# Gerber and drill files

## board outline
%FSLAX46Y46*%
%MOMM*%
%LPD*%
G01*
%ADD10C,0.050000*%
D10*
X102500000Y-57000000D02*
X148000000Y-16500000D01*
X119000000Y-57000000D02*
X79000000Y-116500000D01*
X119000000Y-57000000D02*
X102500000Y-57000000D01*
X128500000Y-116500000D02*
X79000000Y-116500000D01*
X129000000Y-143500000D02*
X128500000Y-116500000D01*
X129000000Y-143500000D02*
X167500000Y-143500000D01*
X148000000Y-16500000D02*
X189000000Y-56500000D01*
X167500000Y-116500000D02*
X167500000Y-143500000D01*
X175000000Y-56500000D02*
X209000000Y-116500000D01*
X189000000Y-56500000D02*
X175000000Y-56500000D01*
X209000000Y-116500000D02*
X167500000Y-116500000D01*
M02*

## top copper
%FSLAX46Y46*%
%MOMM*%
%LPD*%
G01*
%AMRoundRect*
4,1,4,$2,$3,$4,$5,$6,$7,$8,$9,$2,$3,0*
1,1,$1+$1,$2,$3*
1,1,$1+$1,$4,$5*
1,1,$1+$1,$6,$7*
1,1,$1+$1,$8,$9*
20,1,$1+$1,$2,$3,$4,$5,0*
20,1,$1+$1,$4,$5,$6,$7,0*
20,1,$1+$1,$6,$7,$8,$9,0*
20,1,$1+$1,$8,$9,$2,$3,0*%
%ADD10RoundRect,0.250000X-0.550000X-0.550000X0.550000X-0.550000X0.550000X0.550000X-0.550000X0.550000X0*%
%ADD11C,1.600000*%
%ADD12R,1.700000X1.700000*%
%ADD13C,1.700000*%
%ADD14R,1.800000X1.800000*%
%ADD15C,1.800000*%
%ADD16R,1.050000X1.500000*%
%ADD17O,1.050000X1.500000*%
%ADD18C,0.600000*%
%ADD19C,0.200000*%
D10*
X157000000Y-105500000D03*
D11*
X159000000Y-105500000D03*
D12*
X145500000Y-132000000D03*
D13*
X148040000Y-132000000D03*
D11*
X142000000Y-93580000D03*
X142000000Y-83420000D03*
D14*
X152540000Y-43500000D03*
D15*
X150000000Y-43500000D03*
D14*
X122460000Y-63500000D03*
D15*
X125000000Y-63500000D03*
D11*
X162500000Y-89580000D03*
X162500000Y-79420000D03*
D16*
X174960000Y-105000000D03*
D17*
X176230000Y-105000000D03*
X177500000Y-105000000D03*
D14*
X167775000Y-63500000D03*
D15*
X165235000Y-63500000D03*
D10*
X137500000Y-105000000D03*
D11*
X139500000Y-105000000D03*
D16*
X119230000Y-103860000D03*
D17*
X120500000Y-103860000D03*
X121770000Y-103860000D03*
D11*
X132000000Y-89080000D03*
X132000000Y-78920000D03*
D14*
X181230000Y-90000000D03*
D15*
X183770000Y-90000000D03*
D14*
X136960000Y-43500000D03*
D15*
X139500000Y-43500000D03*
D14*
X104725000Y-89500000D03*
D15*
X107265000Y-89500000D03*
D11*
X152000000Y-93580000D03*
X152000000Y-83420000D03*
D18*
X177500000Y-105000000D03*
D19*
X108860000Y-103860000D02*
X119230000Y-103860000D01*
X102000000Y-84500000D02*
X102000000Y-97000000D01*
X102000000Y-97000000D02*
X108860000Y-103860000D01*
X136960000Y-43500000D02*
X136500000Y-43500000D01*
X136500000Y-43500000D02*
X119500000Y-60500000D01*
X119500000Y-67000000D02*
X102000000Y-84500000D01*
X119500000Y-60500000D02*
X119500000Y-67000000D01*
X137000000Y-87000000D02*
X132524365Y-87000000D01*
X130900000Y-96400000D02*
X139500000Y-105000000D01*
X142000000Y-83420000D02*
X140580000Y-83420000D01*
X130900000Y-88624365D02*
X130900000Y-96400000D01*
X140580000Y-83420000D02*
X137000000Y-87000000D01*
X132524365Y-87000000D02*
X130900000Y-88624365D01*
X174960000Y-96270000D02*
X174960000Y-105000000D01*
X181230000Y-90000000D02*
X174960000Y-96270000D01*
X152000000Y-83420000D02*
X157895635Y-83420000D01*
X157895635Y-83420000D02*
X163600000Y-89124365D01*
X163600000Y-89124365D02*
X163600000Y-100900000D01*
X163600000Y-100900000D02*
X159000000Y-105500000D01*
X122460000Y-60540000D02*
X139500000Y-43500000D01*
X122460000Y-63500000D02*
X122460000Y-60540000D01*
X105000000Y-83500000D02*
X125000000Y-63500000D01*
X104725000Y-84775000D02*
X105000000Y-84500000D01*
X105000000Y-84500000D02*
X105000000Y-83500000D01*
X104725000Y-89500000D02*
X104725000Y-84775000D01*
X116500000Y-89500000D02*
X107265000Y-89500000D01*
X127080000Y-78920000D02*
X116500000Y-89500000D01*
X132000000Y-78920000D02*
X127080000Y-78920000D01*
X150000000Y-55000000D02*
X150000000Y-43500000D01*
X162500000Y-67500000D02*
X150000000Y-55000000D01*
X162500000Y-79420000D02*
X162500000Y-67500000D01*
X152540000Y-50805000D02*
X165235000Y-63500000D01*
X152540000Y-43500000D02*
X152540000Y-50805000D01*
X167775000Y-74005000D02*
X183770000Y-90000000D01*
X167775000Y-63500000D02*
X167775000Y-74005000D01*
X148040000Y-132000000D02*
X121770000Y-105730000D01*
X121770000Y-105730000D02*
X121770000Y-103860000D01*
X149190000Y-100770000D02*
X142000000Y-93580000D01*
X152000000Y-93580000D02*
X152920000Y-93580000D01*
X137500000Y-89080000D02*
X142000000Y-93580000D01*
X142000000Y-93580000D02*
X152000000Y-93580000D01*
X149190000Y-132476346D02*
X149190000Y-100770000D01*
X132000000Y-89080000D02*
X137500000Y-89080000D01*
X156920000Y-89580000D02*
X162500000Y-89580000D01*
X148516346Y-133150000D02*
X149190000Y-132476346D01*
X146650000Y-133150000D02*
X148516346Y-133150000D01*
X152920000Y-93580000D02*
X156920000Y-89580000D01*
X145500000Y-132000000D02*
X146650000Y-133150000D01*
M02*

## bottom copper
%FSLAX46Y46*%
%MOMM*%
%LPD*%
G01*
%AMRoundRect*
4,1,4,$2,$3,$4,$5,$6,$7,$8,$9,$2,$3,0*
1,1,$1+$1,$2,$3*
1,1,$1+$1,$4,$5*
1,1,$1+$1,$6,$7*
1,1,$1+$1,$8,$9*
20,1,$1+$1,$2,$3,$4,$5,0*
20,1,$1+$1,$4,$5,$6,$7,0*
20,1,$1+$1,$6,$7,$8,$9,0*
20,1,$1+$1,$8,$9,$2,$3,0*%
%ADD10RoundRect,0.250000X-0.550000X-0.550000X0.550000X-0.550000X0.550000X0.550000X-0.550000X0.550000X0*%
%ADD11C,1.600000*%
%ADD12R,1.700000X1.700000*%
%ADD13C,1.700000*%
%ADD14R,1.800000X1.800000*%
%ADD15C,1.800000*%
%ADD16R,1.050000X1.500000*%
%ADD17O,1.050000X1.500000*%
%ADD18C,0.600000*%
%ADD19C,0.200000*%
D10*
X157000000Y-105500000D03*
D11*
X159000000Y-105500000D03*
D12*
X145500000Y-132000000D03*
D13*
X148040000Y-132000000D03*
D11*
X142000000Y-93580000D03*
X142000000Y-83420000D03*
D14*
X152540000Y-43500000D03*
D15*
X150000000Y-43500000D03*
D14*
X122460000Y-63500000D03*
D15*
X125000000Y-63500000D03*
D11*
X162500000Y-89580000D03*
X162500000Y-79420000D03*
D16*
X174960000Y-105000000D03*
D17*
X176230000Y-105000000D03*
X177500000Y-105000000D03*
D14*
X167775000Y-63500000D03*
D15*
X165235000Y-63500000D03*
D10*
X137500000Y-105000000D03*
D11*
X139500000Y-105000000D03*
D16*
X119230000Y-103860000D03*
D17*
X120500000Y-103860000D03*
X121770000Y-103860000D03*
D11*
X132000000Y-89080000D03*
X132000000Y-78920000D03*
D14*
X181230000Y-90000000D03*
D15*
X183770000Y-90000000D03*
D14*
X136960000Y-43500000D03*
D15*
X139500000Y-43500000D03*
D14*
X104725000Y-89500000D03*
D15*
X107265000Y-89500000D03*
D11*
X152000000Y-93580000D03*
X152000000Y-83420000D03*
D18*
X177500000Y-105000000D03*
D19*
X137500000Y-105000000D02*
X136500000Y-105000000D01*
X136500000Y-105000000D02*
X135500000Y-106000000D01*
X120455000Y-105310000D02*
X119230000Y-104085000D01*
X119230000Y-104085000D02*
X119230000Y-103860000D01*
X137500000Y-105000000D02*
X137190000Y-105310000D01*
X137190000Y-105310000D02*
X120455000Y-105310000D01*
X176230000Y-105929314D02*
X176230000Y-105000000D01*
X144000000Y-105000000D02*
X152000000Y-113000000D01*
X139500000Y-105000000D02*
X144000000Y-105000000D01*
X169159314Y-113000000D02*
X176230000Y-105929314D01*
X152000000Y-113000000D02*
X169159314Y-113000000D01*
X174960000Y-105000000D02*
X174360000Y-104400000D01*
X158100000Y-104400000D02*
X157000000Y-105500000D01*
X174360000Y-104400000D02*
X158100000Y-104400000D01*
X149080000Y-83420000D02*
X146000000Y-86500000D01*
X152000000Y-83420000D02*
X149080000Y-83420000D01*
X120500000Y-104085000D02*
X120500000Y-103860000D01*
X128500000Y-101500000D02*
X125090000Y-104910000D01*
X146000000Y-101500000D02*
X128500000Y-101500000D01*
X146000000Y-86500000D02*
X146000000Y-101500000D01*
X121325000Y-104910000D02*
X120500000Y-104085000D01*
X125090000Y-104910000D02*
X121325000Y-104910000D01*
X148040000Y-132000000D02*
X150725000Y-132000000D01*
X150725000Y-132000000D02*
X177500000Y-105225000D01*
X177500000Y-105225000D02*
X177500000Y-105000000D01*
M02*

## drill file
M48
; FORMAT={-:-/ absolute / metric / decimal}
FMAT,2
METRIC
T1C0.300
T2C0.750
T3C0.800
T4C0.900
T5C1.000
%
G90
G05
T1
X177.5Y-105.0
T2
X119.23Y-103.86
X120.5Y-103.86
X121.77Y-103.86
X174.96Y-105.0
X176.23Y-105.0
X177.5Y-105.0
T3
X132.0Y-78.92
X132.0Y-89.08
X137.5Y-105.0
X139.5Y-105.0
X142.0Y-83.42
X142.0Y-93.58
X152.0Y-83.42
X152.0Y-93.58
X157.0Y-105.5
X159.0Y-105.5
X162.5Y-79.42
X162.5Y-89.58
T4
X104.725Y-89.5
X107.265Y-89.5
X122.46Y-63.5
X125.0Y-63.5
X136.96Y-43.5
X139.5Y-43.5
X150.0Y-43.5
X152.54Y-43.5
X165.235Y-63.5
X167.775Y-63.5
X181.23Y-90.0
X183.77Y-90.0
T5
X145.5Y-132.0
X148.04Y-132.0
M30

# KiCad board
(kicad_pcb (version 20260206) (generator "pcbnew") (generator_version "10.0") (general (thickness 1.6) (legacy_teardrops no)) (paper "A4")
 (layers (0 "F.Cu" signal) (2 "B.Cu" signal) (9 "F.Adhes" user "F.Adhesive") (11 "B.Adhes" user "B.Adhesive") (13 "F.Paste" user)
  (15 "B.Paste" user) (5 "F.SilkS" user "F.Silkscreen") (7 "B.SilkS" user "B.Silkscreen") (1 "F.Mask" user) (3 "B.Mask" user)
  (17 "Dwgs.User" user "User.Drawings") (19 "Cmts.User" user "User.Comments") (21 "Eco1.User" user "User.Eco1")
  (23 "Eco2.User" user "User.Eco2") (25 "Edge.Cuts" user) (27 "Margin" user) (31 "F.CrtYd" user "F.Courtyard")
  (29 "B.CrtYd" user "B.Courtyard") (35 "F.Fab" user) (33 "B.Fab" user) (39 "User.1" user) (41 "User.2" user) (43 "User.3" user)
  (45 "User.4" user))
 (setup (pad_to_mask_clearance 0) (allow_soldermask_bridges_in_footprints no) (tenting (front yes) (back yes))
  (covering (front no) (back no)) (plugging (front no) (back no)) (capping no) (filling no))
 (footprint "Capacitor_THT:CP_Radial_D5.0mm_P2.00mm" (layer "F.Cu") (at 157 105.5)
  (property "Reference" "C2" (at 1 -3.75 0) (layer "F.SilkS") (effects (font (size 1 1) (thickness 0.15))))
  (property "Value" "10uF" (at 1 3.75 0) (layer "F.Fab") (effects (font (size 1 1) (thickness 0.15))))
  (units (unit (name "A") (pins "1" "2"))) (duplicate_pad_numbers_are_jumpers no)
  (pad "1" thru_hole roundrect (at 0 0) (size 1.6 1.6) (drill 0.8) (layers "*.Cu" "*.Mask") (remove_unused_layers no)
   (roundrect_rratio 0.15625) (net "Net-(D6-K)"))
  (pad "2" thru_hole circle (at 2 0) (size 1.6 1.6) (drill 0.8) (layers "*.Cu" "*.Mask") (remove_unused_layers no) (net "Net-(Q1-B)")))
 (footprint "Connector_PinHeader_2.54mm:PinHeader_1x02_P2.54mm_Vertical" (layer "F.Cu") (at 145.5 132 90)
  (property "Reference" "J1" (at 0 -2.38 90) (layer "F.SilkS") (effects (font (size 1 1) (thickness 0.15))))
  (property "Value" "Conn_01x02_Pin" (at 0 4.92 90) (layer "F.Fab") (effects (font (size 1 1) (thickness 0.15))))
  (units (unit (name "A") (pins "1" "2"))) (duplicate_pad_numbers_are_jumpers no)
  (pad "1" thru_hole rect (at 0 0 90) (size 1.7 1.7) (drill 1) (layers "*.Cu" "*.Mask") (remove_unused_layers no) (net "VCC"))
  (pad "2" thru_hole circle (at 0 2.54 90) (size 1.7 1.7) (drill 1) (layers "*.Cu" "*.Mask") (remove_unused_layers no) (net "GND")))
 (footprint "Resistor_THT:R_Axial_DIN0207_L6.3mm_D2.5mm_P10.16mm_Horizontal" (layer "F.Cu") (at 142 93.58 90)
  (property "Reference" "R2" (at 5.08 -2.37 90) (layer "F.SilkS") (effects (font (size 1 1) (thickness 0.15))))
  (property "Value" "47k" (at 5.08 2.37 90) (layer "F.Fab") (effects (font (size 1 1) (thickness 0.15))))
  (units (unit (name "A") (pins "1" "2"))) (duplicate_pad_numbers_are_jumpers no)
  (pad "1" thru_hole circle (at 0 0 90) (size 1.6 1.6) (drill 0.8) (layers "*.Cu" "*.Mask") (remove_unused_layers no) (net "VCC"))
  (pad "2" thru_hole circle (at 10.16 0 90) (size 1.6 1.6) (drill 0.8) (layers "*.Cu" "*.Mask") (remove_unused_layers no) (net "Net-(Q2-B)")))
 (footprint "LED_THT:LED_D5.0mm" (layer "F.Cu") (at 152.54 43.5 180)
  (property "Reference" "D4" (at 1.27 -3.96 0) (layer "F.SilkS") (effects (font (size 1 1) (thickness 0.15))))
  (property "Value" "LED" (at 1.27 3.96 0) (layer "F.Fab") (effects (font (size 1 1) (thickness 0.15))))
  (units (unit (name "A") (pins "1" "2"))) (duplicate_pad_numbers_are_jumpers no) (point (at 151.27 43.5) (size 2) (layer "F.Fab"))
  (pad "1" thru_hole rect (at 0 0 180) (size 1.8 1.8) (drill 0.9) (layers "*.Cu" "*.Mask") (remove_unused_layers no) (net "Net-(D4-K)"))
  (pad "2" thru_hole circle (at 2.54 0 180) (size 1.8 1.8) (drill 0.9) (layers "*.Cu" "*.Mask") (remove_unused_layers no) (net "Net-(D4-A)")))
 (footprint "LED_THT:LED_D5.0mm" (layer "F.Cu") (at 122.46 63.5)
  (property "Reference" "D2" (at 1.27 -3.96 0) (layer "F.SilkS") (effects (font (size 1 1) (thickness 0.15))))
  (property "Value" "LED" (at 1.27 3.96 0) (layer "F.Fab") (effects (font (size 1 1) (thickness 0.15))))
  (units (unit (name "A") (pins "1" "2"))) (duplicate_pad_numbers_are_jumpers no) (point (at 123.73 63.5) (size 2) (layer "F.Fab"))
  (pad "1" thru_hole rect (at 0 0) (size 1.8 1.8) (drill 0.9) (layers "*.Cu" "*.Mask") (remove_unused_layers no) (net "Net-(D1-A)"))
  (pad "2" thru_hole circle (at 2.54 0) (size 1.8 1.8) (drill 0.9) (layers "*.Cu" "*.Mask") (remove_unused_layers no) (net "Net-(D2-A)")))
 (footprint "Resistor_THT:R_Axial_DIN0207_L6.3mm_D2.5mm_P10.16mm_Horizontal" (layer "F.Cu") (at 162.5 89.58 90)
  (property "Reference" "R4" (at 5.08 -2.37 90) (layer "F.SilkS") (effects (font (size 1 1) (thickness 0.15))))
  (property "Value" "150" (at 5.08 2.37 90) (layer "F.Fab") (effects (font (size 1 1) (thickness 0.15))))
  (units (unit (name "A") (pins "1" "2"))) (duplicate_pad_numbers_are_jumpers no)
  (pad "1" thru_hole circle (at 0 0 90) (size 1.6 1.6) (drill 0.8) (layers "*.Cu" "*.Mask") (remove_unused_layers no) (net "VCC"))
  (pad "2" thru_hole circle (at 10.16 0 90) (size 1.6 1.6) (drill 0.8) (layers "*.Cu" "*.Mask") (remove_unused_layers no) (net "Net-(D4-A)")))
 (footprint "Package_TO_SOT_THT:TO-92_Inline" (layer "F.Cu") (at 174.96 105)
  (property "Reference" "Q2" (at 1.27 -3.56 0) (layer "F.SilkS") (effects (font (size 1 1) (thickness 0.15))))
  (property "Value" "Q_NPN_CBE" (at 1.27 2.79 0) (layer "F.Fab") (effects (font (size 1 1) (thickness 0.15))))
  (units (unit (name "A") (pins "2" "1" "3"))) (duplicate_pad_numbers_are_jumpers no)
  (pad "1" thru_hole rect (at 0 0) (size 1.05 1.5) (drill 0.75) (layers "*.Cu" "*.Mask") (remove_unused_layers no) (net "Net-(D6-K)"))
  (pad "2" thru_hole oval (at 1.27 0) (size 1.05 1.5) (drill 0.75) (layers "*.Cu" "*.Mask") (remove_unused_layers no) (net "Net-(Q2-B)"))
  (pad "3" thru_hole oval (at 2.54 0) (size 1.05 1.5) (drill 0.75) (layers "*.Cu" "*.Mask") (remove_unused_layers no) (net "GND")))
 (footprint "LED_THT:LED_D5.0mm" (layer "F.Cu") (at 167.775 63.5 180)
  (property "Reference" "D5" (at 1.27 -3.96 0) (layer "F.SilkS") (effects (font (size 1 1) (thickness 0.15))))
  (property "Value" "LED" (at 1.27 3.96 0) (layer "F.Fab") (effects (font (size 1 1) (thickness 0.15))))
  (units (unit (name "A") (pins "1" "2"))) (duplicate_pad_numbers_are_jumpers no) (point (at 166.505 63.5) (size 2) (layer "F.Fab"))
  (pad "1" thru_hole rect (at 0 0 180) (size 1.8 1.8) (drill 0.9) (layers "*.Cu" "*.Mask") (remove_unused_layers no) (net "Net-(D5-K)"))
  (pad "2" thru_hole circle (at 2.54 0 180) (size 1.8 1.8) (drill 0.9) (layers "*.Cu" "*.Mask") (remove_unused_layers no) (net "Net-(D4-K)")))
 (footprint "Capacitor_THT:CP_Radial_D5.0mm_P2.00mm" (layer "F.Cu") (at 137.5 105)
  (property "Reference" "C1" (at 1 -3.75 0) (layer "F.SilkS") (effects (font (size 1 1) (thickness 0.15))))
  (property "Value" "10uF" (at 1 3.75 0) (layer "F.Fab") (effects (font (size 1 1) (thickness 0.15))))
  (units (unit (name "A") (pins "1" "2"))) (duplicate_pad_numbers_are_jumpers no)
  (pad "1" thru_hole roundrect (at 0 0) (size 1.6 1.6) (drill 0.8) (layers "*.Cu" "*.Mask") (remove_unused_layers no)
   (roundrect_rratio 0.15625) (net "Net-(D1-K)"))
  (pad "2" thru_hole circle (at 2 0) (size 1.6 1.6) (drill 0.8) (layers "*.Cu" "*.Mask") (remove_unused_layers no) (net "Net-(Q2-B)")))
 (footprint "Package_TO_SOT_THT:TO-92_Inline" (layer "F.Cu") (at 119.23 103.86)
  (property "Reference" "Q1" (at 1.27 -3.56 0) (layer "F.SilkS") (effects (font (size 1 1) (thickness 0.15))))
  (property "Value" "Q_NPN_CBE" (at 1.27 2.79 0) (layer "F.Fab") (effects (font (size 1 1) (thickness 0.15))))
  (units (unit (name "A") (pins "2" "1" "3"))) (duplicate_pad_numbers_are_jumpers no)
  (pad "1" thru_hole rect (at 0 0) (size 1.05 1.5) (drill 0.75) (layers "*.Cu" "*.Mask") (remove_unused_layers no) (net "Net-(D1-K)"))
  (pad "2" thru_hole oval (at 1.27 0) (size 1.05 1.5) (drill 0.75) (layers "*.Cu" "*.Mask") (remove_unused_layers no) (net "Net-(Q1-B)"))
  (pad "3" thru_hole oval (at 2.54 0) (size 1.05 1.5) (drill 0.75) (layers "*.Cu" "*.Mask") (remove_unused_layers no) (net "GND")))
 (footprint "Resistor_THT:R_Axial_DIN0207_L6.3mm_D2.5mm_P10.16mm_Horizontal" (layer "F.Cu") (at 132 89.08 90)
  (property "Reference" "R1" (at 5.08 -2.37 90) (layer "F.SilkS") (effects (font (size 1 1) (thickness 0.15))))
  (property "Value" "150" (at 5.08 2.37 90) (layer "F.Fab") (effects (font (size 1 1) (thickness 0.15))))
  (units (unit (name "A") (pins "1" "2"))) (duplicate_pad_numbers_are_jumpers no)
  (pad "1" thru_hole circle (at 0 0 90) (size 1.6 1.6) (drill 0.8) (layers "*.Cu" "*.Mask") (remove_unused_layers no) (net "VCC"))
  (pad "2" thru_hole circle (at 10.16 0 90) (size 1.6 1.6) (drill 0.8) (layers "*.Cu" "*.Mask") (remove_unused_layers no) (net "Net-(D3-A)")))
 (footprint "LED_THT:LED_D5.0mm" (layer "F.Cu") (at 181.23 90)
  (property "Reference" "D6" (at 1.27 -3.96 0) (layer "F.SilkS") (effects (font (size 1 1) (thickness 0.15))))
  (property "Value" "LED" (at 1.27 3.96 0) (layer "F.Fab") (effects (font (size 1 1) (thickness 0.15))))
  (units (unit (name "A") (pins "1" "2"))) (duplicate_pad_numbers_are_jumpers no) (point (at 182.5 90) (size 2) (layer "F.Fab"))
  (pad "1" thru_hole rect (at 0 0) (size 1.8 1.8) (drill 0.9) (layers "*.Cu" "*.Mask") (remove_unused_layers no) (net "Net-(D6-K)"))
  (pad "2" thru_hole circle (at 2.54 0) (size 1.8 1.8) (drill 0.9) (layers "*.Cu" "*.Mask") (remove_unused_layers no) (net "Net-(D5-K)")))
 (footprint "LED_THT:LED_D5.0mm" (layer "F.Cu") (at 136.96 43.5)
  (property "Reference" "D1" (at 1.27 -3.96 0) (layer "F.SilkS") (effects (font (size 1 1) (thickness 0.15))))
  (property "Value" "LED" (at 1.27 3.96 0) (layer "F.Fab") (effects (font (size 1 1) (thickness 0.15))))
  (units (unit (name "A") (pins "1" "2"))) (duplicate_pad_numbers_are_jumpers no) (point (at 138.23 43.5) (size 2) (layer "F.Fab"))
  (pad "1" thru_hole rect (at 0 0) (size 1.8 1.8) (drill 0.9) (layers "*.Cu" "*.Mask") (remove_unused_layers no) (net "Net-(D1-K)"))
  (pad "2" thru_hole circle (at 2.54 0) (size 1.8 1.8) (drill 0.9) (layers "*.Cu" "*.Mask") (remove_unused_layers no) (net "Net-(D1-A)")))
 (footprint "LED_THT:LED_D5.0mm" (layer "F.Cu") (at 104.725 89.5)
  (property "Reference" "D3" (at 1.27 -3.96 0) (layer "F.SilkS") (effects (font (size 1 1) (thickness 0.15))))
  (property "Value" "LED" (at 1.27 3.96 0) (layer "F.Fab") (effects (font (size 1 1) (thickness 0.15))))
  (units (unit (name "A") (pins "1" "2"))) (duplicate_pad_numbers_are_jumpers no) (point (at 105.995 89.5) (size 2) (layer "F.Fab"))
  (pad "1" thru_hole rect (at 0 0) (size 1.8 1.8) (drill 0.9) (layers "*.Cu" "*.Mask") (remove_unused_layers no) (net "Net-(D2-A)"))
  (pad "2" thru_hole circle (at 2.54 0) (size 1.8 1.8) (drill 0.9) (layers "*.Cu" "*.Mask") (remove_unused_layers no) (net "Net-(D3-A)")))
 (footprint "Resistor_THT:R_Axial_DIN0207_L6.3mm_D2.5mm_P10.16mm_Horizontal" (layer "F.Cu") (at 152 93.58 90)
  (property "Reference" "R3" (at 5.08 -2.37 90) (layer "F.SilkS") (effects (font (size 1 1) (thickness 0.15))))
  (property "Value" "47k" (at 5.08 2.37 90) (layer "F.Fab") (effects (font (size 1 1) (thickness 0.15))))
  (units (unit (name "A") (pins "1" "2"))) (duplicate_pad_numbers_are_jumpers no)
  (pad "1" thru_hole circle (at 0 0 90) (size 1.6 1.6) (drill 0.8) (layers "*.Cu" "*.Mask") (remove_unused_layers no) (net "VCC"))
  (pad "2" thru_hole circle (at 10.16 0 90) (size 1.6 1.6) (drill 0.8) (layers "*.Cu" "*.Mask") (remove_unused_layers no) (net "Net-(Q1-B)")))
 (gr_line (start 102.5 57) (end 148 16.5) (stroke (width 0.05) (type default)) (layer "Edge.Cuts"))
 (gr_line (start 119 57) (end 79 116.5) (stroke (width 0.05) (type default)) (layer "Edge.Cuts"))
 (gr_line (start 119 57) (end 102.5 57) (stroke (width 0.05) (type default)) (layer "Edge.Cuts"))
 (gr_line (start 128.5 116.5) (end 79 116.5) (stroke (width 0.05) (type default)) (layer "Edge.Cuts"))
 (gr_line (start 129 143.5) (end 128.5 116.5) (stroke (width 0.05) (type default)) (layer "Edge.Cuts"))
 (gr_line (start 129 143.5) (end 167.5 143.5) (stroke (width 0.05) (type default)) (layer "Edge.Cuts"))
 (gr_line (start 148 16.5) (end 189 56.5) (stroke (width 0.05) (type default)) (layer "Edge.Cuts"))
 (gr_line (start 167.5 116.5) (end 167.5 143.5) (stroke (width 0.05) (type default)) (layer "Edge.Cuts"))
 (gr_line (start 175 56.5) (end 209 116.5) (stroke (width 0.05) (type default)) (layer "Edge.Cuts"))
 (gr_line (start 189 56.5) (end 175 56.5) (stroke (width 0.05) (type default)) (layer "Edge.Cuts"))
 (gr_line (start 209 116.5) (end 167.5 116.5) (stroke (width 0.05) (type default)) (layer "Edge.Cuts"))
 (segment (start 108.86 103.86) (end 119.23 103.86) (width 0.2) (layer "F.Cu") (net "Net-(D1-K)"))
 (segment (start 102 84.5) (end 102 97) (width 0.2) (layer "F.Cu") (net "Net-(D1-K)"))
 (segment (start 102 97) (end 108.86 103.86) (width 0.2) (layer "F.Cu") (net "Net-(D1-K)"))
 (segment (start 136.96 43.5) (end 136.5 43.5) (width 0.2) (layer "F.Cu") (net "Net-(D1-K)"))
 (segment (start 136.5 43.5) (end 119.5 60.5) (width 0.2) (layer "F.Cu") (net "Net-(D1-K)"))
 (segment (start 119.5 67) (end 102 84.5) (width 0.2) (layer "F.Cu") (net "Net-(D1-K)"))
 (segment (start 119.5 60.5) (end 119.5 67) (width 0.2) (layer "F.Cu") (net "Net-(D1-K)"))
 (segment (start 137.5 105) (end 136.5 105) (width 0.2) (layer "B.Cu") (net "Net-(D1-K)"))
 (segment (start 136.5 105) (end 135.5 106) (width 0.2) (layer "B.Cu") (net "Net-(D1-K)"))
 (segment (start 120.455 105.31) (end 119.23 104.085) (width 0.2) (layer "B.Cu") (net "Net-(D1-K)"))
 (segment (start 119.23 104.085) (end 119.23 103.86) (width 0.2) (layer "B.Cu") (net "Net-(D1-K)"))
 (segment (start 137.5 105) (end 137.19 105.31) (width 0.2) (layer "B.Cu") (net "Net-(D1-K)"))
 (segment (start 137.19 105.31) (end 120.455 105.31) (width 0.2) (layer "B.Cu") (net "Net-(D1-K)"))
 (segment (start 137 87) (end 132.524365 87) (width 0.2) (layer "F.Cu") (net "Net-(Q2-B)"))
 (segment (start 130.9 96.4) (end 139.5 105) (width 0.2) (layer "F.Cu") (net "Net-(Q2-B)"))
 (segment (start 142 83.42) (end 140.58 83.42) (width 0.2) (layer "F.Cu") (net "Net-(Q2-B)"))
 (segment (start 130.9 88.624365) (end 130.9 96.4) (width 0.2) (layer "F.Cu") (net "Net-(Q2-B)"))
 (segment (start 140.58 83.42) (end 137 87) (width 0.2) (layer "F.Cu") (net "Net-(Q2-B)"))
 (segment (start 132.524365 87) (end 130.9 88.624365) (width 0.2) (layer "F.Cu") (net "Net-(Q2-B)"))
 (segment (start 176.23 105.929314) (end 176.23 105) (width 0.2) (layer "B.Cu") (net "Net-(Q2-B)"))
 (segment (start 144 105) (end 152 113) (width 0.2) (layer "B.Cu") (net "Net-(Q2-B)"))
 (segment (start 139.5 105) (end 144 105) (width 0.2) (layer "B.Cu") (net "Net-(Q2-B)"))
 (segment (start 169.159314 113) (end 176.23 105.929314) (width 0.2) (layer "B.Cu") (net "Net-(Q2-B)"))
 (segment (start 152 113) (end 169.159314 113) (width 0.2) (layer "B.Cu") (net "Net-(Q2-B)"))
 (segment (start 174.96 96.27) (end 174.96 105) (width 0.2) (layer "F.Cu") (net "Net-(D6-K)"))
 (segment (start 181.23 90) (end 174.96 96.27) (width 0.2) (layer "F.Cu") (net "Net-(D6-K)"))
 (segment (start 174.96 105) (end 174.36 104.4) (width 0.2) (layer "B.Cu") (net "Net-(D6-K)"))
 (segment (start 158.1 104.4) (end 157 105.5) (width 0.2) (layer "B.Cu") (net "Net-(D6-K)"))
 (segment (start 174.36 104.4) (end 158.1 104.4) (width 0.2) (layer "B.Cu") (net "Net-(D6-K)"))
 (segment (start 152 83.42) (end 157.895635 83.42) (width 0.2) (layer "F.Cu") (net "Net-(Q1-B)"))
 (segment (start 157.895635 83.42) (end 163.6 89.124365) (width 0.2) (layer "F.Cu") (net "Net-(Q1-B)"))
 (segment (start 163.6 89.124365) (end 163.6 100.9) (width 0.2) (layer "F.Cu") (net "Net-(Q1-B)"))
 (segment (start 163.6 100.9) (end 159 105.5) (width 0.2) (layer "F.Cu") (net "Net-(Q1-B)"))
 (segment (start 149.08 83.42) (end 146 86.5) (width 0.2) (layer "B.Cu") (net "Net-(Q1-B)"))
 (segment (start 152 83.42) (end 149.08 83.42) (width 0.2) (layer "B.Cu") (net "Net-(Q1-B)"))
 (segment (start 120.5 104.085) (end 120.5 103.86) (width 0.2) (layer "B.Cu") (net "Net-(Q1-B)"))
 (segment (start 128.5 101.5) (end 125.09 104.91) (width 0.2) (layer "B.Cu") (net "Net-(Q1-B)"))
 (segment (start 146 101.5) (end 128.5 101.5) (width 0.2) (layer "B.Cu") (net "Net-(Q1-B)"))
 (segment (start 146 86.5) (end 146 101.5) (width 0.2) (layer "B.Cu") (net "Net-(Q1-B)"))
 (segment (start 121.325 104.91) (end 120.5 104.085) (width 0.2) (layer "B.Cu") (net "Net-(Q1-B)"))
 (segment (start 125.09 104.91) (end 121.325 104.91) (width 0.2) (layer "B.Cu") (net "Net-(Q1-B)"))
 (segment (start 122.46 60.54) (end 139.5 43.5) (width 0.2) (layer "F.Cu") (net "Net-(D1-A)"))
 (segment (start 122.46 63.5) (end 122.46 60.54) (width 0.2) (layer "F.Cu") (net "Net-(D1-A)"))
 (segment (start 105 83.5) (end 125 63.5) (width 0.2) (layer "F.Cu") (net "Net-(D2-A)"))
 (segment (start 104.725 84.775) (end 105 84.5) (width 0.2) (layer "F.Cu") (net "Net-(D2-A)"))
 (segment (start 105 84.5) (end 105 83.5) (width 0.2) (layer "F.Cu") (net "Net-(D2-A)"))
 (segment (start 104.725 89.5) (end 104.725 84.775) (width 0.2) (layer "F.Cu") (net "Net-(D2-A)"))
 (segment (start 116.5 89.5) (end 107.265 89.5) (width 0.2) (layer "F.Cu") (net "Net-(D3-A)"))
 (segment (start 127.08 78.92) (end 116.5 89.5) (width 0.2) (layer "F.Cu") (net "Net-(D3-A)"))
 (segment (start 132 78.92) (end 127.08 78.92) (width 0.2) (layer "F.Cu") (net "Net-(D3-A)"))
 (segment (start 150 55) (end 150 43.5) (width 0.2) (layer "F.Cu") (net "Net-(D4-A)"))
 (segment (start 162.5 67.5) (end 150 55) (width 0.2) (layer "F.Cu") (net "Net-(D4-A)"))
 (segment (start 162.5 79.42) (end 162.5 67.5) (width 0.2) (layer "F.Cu") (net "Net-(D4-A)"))
 (segment (start 152.54 50.805) (end 165.235 63.5) (width 0.2) (layer "F.Cu") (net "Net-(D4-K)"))
 (segment (start 152.54 43.5) (end 152.54 50.805) (width 0.2) (layer "F.Cu") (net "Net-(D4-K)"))
 (segment (start 167.775 74.005) (end 183.77 90) (width 0.2) (layer "F.Cu") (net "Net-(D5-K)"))
 (segment (start 167.775 63.5) (end 167.775 74.005) (width 0.2) (layer "F.Cu") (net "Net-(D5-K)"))
 (segment (start 148.04 132) (end 121.77 105.73) (width 0.2) (layer "F.Cu") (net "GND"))
 (segment (start 121.77 105.73) (end 121.77 103.86) (width 0.2) (layer "F.Cu") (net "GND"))
 (via (at 177.5 105) (size 0.6) (drill 0.3) (layers "F.Cu" "B.Cu") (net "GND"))
 (segment (start 148.04 132) (end 150.725 132) (width 0.2) (layer "B.Cu") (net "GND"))
 (segment (start 150.725 132) (end 177.5 105.225) (width 0.2) (layer "B.Cu") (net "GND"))
 (segment (start 177.5 105.225) (end 177.5 105) (width 0.2) (layer "B.Cu") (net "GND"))
 (segment (start 149.19 100.77) (end 142 93.58) (width 0.2) (layer "F.Cu") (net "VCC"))
 (segment (start 152 93.58) (end 152.92 93.58) (width 0.2) (layer "F.Cu") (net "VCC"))
 (segment (start 137.5 89.08) (end 142 93.58) (width 0.2) (layer "F.Cu") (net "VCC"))
 (segment (start 142 93.58) (end 152 93.58) (width 0.2) (layer "F.Cu") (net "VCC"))
 (segment (start 149.19 132.476346) (end 149.19 100.77) (width 0.2) (layer "F.Cu") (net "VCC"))
 (segment (start 132 89.08) (end 137.5 89.08) (width 0.2) (layer "F.Cu") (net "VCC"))
 (segment (start 156.92 89.58) (end 162.5 89.58) (width 0.2) (layer "F.Cu") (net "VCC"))
 (segment (start 148.516346 133.15) (end 149.19 132.476346) (width 0.2) (layer "F.Cu") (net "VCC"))
 (segment (start 146.65 133.15) (end 148.516346 133.15) (width 0.2) (layer "F.Cu") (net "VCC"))
 (segment (start 152.92 93.58) (end 156.92 89.58) (width 0.2) (layer "F.Cu") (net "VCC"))
 (segment (start 145.5 132) (end 146.65 133.15) (width 0.2) (layer "F.Cu") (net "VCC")))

